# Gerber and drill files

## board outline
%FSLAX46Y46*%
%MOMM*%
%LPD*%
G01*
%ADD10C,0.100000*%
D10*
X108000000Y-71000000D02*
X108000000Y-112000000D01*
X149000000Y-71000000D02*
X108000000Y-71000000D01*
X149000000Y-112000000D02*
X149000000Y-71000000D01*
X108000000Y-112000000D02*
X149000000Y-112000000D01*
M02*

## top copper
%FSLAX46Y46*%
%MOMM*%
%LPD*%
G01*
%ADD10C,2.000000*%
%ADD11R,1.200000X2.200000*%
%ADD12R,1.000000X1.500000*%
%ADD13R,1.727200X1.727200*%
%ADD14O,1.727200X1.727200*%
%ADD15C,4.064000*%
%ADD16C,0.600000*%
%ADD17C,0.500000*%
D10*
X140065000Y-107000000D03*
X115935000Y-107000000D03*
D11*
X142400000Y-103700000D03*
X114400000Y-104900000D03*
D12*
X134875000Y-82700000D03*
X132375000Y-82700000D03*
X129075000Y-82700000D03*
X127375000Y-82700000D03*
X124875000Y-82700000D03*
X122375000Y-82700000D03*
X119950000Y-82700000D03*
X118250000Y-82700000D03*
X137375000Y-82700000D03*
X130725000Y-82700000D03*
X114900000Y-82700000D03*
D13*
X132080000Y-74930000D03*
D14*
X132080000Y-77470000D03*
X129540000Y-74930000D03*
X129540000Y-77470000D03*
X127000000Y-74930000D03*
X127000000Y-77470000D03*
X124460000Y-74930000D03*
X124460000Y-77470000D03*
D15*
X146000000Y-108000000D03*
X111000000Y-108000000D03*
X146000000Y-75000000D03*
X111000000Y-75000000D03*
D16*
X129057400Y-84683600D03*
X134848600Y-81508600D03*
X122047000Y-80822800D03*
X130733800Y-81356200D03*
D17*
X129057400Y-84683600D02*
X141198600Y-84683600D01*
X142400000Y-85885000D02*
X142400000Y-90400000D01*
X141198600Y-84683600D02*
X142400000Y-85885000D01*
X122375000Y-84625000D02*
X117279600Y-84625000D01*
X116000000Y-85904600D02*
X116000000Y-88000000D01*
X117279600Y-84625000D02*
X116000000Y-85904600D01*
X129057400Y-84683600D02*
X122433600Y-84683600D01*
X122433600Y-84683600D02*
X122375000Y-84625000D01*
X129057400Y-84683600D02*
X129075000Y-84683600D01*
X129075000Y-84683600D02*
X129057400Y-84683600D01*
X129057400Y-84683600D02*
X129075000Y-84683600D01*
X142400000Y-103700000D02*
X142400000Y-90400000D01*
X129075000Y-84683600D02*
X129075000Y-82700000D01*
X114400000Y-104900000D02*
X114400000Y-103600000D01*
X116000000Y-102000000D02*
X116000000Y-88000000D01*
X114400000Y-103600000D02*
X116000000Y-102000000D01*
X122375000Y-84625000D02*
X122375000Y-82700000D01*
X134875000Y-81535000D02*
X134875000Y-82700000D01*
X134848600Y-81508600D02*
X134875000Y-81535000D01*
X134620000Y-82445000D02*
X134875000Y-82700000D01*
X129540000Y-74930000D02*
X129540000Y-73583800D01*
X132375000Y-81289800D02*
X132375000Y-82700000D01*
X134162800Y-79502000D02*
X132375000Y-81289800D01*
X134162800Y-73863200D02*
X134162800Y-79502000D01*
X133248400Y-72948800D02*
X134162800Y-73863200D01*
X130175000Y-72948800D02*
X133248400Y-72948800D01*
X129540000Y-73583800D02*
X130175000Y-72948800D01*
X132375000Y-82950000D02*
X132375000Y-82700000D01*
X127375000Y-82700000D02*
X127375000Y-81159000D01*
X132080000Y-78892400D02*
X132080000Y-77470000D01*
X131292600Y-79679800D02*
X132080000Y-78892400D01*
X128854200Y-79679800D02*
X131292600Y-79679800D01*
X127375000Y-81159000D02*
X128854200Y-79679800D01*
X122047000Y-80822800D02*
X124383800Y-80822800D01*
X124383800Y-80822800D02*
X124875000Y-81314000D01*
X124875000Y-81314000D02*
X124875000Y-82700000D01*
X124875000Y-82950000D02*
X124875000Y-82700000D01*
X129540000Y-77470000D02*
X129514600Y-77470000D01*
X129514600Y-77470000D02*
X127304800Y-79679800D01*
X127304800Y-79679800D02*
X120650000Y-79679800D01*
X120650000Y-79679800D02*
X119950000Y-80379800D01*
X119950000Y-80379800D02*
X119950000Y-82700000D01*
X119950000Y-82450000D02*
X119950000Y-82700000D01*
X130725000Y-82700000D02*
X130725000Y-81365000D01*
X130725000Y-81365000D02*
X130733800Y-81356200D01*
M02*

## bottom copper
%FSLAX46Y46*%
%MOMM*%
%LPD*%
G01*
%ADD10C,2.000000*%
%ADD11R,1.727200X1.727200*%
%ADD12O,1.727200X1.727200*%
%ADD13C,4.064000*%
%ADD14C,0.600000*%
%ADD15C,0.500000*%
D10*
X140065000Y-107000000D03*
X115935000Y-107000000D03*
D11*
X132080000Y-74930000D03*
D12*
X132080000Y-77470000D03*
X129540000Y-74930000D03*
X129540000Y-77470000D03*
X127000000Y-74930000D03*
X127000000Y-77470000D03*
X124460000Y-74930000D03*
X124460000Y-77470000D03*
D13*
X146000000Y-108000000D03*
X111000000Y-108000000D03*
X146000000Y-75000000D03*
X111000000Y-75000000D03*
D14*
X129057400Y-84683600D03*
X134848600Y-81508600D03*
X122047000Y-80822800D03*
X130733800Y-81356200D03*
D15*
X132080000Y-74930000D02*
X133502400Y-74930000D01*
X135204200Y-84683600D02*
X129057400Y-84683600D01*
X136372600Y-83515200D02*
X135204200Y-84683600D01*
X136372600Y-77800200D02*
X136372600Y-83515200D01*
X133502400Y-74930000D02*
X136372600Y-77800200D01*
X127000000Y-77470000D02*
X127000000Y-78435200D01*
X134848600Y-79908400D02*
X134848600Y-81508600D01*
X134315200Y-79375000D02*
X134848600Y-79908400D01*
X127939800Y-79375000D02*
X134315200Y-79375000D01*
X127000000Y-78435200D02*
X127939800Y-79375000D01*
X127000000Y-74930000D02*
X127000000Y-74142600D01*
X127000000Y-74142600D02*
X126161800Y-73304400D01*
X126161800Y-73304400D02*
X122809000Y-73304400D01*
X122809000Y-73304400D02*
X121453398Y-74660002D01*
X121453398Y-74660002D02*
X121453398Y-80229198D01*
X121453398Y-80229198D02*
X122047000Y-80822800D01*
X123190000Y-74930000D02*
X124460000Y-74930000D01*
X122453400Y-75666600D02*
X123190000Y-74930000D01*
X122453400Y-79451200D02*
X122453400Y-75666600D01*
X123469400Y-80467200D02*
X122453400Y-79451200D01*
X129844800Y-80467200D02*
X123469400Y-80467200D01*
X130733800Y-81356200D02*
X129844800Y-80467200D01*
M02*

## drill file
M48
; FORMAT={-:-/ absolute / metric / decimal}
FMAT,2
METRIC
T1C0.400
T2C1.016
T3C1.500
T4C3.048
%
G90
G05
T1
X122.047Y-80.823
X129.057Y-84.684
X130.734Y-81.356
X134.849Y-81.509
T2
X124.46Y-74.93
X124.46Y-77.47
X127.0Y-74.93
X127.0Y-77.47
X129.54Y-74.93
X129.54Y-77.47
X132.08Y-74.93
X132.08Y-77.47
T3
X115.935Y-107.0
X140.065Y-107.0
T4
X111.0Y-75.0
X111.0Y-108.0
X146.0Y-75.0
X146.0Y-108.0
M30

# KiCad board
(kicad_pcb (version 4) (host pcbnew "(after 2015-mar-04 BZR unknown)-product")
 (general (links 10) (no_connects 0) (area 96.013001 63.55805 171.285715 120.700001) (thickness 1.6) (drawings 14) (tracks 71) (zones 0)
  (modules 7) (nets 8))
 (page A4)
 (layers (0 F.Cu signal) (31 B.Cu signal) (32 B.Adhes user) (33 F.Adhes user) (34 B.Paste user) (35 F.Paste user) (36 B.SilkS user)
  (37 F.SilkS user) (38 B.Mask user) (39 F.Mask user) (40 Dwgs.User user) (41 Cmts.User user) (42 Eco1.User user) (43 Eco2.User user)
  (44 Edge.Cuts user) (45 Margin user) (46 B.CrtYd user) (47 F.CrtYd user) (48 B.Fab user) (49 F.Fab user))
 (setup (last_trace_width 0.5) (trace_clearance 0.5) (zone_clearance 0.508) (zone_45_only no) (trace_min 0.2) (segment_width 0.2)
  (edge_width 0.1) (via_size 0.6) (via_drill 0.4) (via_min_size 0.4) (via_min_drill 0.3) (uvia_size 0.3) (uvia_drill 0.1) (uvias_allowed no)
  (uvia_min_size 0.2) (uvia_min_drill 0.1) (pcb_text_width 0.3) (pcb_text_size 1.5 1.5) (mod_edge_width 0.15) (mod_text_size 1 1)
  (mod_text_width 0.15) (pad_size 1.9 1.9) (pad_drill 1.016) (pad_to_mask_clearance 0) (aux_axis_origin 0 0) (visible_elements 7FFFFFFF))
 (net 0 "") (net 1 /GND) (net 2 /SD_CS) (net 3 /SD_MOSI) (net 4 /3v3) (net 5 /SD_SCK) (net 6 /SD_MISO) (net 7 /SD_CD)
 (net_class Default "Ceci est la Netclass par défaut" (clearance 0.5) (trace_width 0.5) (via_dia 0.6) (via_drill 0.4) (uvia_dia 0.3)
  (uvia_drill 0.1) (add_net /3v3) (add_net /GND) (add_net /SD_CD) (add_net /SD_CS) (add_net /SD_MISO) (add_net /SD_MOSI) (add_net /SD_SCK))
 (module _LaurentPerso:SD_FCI (layer F.Cu) (at 128 107)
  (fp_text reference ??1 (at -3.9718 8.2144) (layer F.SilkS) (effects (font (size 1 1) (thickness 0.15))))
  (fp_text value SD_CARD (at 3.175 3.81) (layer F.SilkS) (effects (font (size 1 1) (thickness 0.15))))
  (pad "" thru_hole circle (at 12.065 0) (size 2 2) (drill 1.5) (layers *.Cu *.Mask F.SilkS))
  (pad "" thru_hole circle (at -12.065 0) (size 2 2) (drill 1.5) (layers *.Cu *.Mask F.SilkS))
  (pad GND smd rect (at 14.4 -3.3) (size 1.2 2.2) (layers F.Cu F.Paste F.Mask) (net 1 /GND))
  (pad GND smd rect (at -13.6 -2.1) (size 1.2 2.2) (layers F.Cu F.Paste F.Mask) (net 1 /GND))
  (pad 1 smd rect (at 6.875 -24.3) (size 1 1.5) (layers F.Cu F.Paste F.Mask) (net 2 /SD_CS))
  (pad 2 smd rect (at 4.375 -24.3) (size 1 1.5) (layers F.Cu F.Paste F.Mask) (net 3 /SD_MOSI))
  (pad 3 smd rect (at 1.075 -24.3) (size 1 1.5) (layers F.Cu F.Paste F.Mask) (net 1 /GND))
  (pad 4 smd rect (at -0.625 -24.3) (size 1 1.5) (layers F.Cu F.Paste F.Mask) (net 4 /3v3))
  (pad 5 smd rect (at -3.125 -24.3) (size 1 1.5) (layers F.Cu F.Paste F.Mask) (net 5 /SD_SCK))
  (pad 6 smd rect (at -5.625 -24.3) (size 1 1.5) (layers F.Cu F.Paste F.Mask) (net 1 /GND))
  (pad 7 smd rect (at -8.05 -24.3) (size 1 1.5) (layers F.Cu F.Paste F.Mask) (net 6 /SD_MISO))
  (pad 8 smd rect (at -9.75 -24.3) (size 1 1.5) (layers F.Cu F.Paste F.Mask))
  (pad 9 smd rect (at 9.375 -24.3) (size 1 1.5) (layers F.Cu F.Paste F.Mask))
  (pad CD smd rect (at 2.725 -24.3) (size 1 1.5) (layers F.Cu F.Paste F.Mask) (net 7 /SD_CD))
  (pad WP smd rect (at -13.1 -24.3) (size 1 1.5) (layers F.Cu F.Paste F.Mask)))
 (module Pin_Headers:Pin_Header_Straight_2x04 (layer F.Cu) (at 132.08 74.93 270)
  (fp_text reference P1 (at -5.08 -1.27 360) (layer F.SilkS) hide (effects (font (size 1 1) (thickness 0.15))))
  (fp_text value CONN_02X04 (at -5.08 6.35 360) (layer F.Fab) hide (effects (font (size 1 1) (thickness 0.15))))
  (pad 1 thru_hole rect (at 0 0 270) (size 1.7272 1.7272) (drill 1.016) (layers *.Cu *.Mask F.SilkS) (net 1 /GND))
  (pad 2 thru_hole oval (at 2.54 0 270) (size 1.7272 1.7272) (drill 1.016) (layers *.Cu *.Mask F.SilkS) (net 4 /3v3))
  (pad 3 thru_hole oval (at 0 2.54 270) (size 1.7272 1.7272) (drill 1.016) (layers *.Cu *.Mask F.SilkS) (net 3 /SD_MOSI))
  (pad 4 thru_hole oval (at 2.54 2.54 270) (size 1.7272 1.7272) (drill 1.016) (layers *.Cu *.Mask F.SilkS) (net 6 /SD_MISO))
  (pad 5 thru_hole oval (at 0 5.08 270) (size 1.7272 1.7272) (drill 1.016) (layers *.Cu *.Mask F.SilkS) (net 5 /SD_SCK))
  (pad 6 thru_hole oval (at 2.54 5.08 270) (size 1.7272 1.7272) (drill 1.016) (layers *.Cu *.Mask F.SilkS) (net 2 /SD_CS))
  (pad 7 thru_hole oval (at 0 7.62 270) (size 1.7272 1.7272) (drill 1.016) (layers *.Cu *.Mask F.SilkS) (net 7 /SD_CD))
  (pad 8 thru_hole oval (at 2.54 7.62 270) (size 1.7272 1.7272) (drill 1.016) (layers *.Cu *.Mask F.SilkS)))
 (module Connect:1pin (layer F.Cu) (at 146 108)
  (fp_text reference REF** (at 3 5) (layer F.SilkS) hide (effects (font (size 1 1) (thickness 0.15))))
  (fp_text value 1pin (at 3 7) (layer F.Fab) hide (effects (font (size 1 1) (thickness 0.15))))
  (pad 1 thru_hole circle (at 0 0) (size 4.064 4.064) (drill 3.048) (layers *.Cu *.Mask F.SilkS)))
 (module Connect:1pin (layer F.Cu) (at 111 108)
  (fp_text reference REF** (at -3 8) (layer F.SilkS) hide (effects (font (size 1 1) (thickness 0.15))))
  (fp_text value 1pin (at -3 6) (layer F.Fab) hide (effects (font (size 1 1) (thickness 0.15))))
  (pad 1 thru_hole circle (at 0 0) (size 4.064 4.064) (drill 3.048) (layers *.Cu *.Mask F.SilkS)))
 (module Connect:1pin (layer F.Cu) (at 146 75)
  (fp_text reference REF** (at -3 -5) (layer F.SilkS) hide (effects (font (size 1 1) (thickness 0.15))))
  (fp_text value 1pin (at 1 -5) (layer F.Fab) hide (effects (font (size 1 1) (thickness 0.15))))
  (pad 1 thru_hole circle (at 0 0) (size 4.064 4.064) (drill 3.048) (layers *.Cu *.Mask F.SilkS)))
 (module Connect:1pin (layer F.Cu) (at 111 75)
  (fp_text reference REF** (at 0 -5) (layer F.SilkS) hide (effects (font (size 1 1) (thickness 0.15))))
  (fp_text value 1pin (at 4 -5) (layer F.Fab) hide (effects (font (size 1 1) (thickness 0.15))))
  (pad 1 thru_hole circle (at 0 0) (size 4.064 4.064) (drill 3.048) (layers *.Cu *.Mask F.SilkS)))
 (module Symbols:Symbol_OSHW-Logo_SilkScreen (layer F.Cu) (at 128.016 95.631)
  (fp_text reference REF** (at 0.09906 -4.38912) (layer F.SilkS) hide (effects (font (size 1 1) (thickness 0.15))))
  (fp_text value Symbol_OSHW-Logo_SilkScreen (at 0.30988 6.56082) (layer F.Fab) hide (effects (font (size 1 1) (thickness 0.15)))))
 (gr_line (start 108 71) (end 108 112) (angle 90) (layer Edge.Cuts) (width 0.1))
 (gr_line (start 149 71) (end 108 71) (angle 90) (layer Edge.Cuts) (width 0.1))
 (gr_line (start 149 112) (end 149 71) (angle 90) (layer Edge.Cuts) (width 0.1))
 (gr_line (start 108 112) (end 149 112) (angle 90) (layer Edge.Cuts) (width 0.1))
 (segment (start 129.0574 84.6836) (end 141.1986 84.6836) (width 0.5) (layer F.Cu) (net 1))
 (segment (start 142.4 85.885) (end 142.4 90.4) (width 0.5) (layer F.Cu) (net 1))
 (segment (start 141.1986 84.6836) (end 142.4 85.885) (width 0.5) (layer F.Cu) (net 1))
 (segment (start 122.375 84.625) (end 117.2796 84.625) (width 0.5) (layer F.Cu) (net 1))
 (segment (start 116 85.9046) (end 116 88) (width 0.5) (layer F.Cu) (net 1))
 (segment (start 117.2796 84.625) (end 116 85.9046) (width 0.5) (layer F.Cu) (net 1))
 (segment (start 129.0574 84.6836) (end 122.4336 84.6836) (width 0.5) (layer F.Cu) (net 1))
 (segment (start 122.4336 84.6836) (end 122.375 84.625) (width 0.5) (layer F.Cu) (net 1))
 (segment (start 132.08 74.93) (end 133.5024 74.93) (width 0.5) (layer B.Cu) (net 1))
 (via (at 129.0574 84.6836) (size 0.6) (layers F.Cu B.Cu) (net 1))
 (segment (start 135.2042 84.6836) (end 129.0574 84.6836) (width 0.5) (layer B.Cu) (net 1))
 (segment (start 136.3726 83.5152) (end 135.2042 84.6836) (width 0.5) (layer B.Cu) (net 1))
 (segment (start 136.3726 77.8002) (end 136.3726 83.5152) (width 0.5) (layer B.Cu) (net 1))
 (segment (start 133.5024 74.93) (end 136.3726 77.8002) (width 0.5) (layer B.Cu) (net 1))
 (segment (start 129.0574 84.6836) (end 129.075 84.6836) (width 0.5) (layer F.Cu) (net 1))
 (segment (start 129.075 84.6836) (end 129.0574 84.6836) (width 0.5) (layer F.Cu) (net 1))
 (segment (start 129.0574 84.6836) (end 129.075 84.6836) (width 0.5) (layer F.Cu) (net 1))
 (segment (start 142.4 103.7) (end 142.4 90.4) (width 0.5) (layer F.Cu) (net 1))
 (segment (start 129.075 84.6836) (end 129.075 82.7) (width 0.5) (layer F.Cu) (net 1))
 (segment (start 114.4 104.9) (end 114.4 103.6) (width 0.5) (layer F.Cu) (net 1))
 (segment (start 116 102) (end 116 88) (width 0.5) (layer F.Cu) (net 1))
 (segment (start 114.4 103.6) (end 116 102) (width 0.5) (layer F.Cu) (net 1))
 (segment (start 122.375 84.625) (end 122.375 82.7) (width 0.5) (layer F.Cu) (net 1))
 (segment (start 127 77.47) (end 127 78.4352) (width 0.5) (layer B.Cu) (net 2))
 (segment (start 134.875 81.535) (end 134.875 82.7) (width 0.5) (layer F.Cu) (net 2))
 (segment (start 134.8486 81.5086) (end 134.875 81.535) (width 0.5) (layer F.Cu) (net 2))
 (via (at 134.8486 81.5086) (size 0.6) (layers F.Cu B.Cu) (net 2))
 (segment (start 134.8486 79.9084) (end 134.8486 81.5086) (width 0.5) (layer B.Cu) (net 2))
 (segment (start 134.3152 79.375) (end 134.8486 79.9084) (width 0.5) (layer B.Cu) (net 2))
 (segment (start 127.9398 79.375) (end 134.3152 79.375) (width 0.5) (layer B.Cu) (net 2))
 (segment (start 127 78.4352) (end 127.9398 79.375) (width 0.5) (layer B.Cu) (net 2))
 (segment (start 134.62 82.445) (end 134.875 82.7) (width 0.5) (layer F.Cu) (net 2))
 (segment (start 129.54 74.93) (end 129.54 73.5838) (width 0.5) (layer F.Cu) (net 3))
 (segment (start 132.375 81.2898) (end 132.375 82.7) (width 0.5) (layer F.Cu) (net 3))
 (segment (start 134.1628 79.502) (end 132.375 81.2898) (width 0.5) (layer F.Cu) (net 3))
 (segment (start 134.1628 73.8632) (end 134.1628 79.502) (width 0.5) (layer F.Cu) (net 3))
 (segment (start 133.2484 72.9488) (end 134.1628 73.8632) (width 0.5) (layer F.Cu) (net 3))
 (segment (start 130.175 72.9488) (end 133.2484 72.9488) (width 0.5) (layer F.Cu) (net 3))
 (segment (start 129.54 73.5838) (end 130.175 72.9488) (width 0.5) (layer F.Cu) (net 3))
 (segment (start 132.375 82.95) (end 132.375 82.7) (width 0.5) (layer F.Cu) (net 3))
 (segment (start 127.375 82.7) (end 127.375 81.159) (width 0.5) (layer F.Cu) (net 4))
 (segment (start 132.08 78.8924) (end 132.08 77.47) (width 0.5) (layer F.Cu) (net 4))
 (segment (start 131.2926 79.6798) (end 132.08 78.8924) (width 0.5) (layer F.Cu) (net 4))
 (segment (start 128.8542 79.6798) (end 131.2926 79.6798) (width 0.5) (layer F.Cu) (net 4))
 (segment (start 127.375 81.159) (end 128.8542 79.6798) (width 0.5) (layer F.Cu) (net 4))
 (segment (start 127 74.93) (end 127 74.1426) (width 0.5) (layer B.Cu) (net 5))
 (segment (start 127 74.1426) (end 126.1618 73.3044) (width 0.5) (layer B.Cu) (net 5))
 (segment (start 126.1618 73.3044) (end 122.809 73.3044) (width 0.5) (layer B.Cu) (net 5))
 (segment (start 122.809 73.3044) (end 121.453398 74.660002) (width 0.5) (layer B.Cu) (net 5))
 (segment (start 121.453398 74.660002) (end 121.453398 80.229198) (width 0.5) (layer B.Cu) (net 5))
 (segment (start 121.453398 80.229198) (end 122.047 80.8228) (width 0.5) (layer B.Cu) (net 5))
 (via (at 122.047 80.8228) (size 0.6) (layers F.Cu B.Cu) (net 5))
 (segment (start 122.047 80.8228) (end 124.3838 80.8228) (width 0.5) (layer F.Cu) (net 5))
 (segment (start 124.3838 80.8228) (end 124.875 81.314) (width 0.5) (layer F.Cu) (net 5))
 (segment (start 124.875 81.314) (end 124.875 82.7) (width 0.5) (layer F.Cu) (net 5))
 (segment (start 124.875 82.95) (end 124.875 82.7) (width 0.5) (layer F.Cu) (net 5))
 (segment (start 129.54 77.47) (end 129.5146 77.47) (width 0.5) (layer F.Cu) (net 6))
 (segment (start 129.5146 77.47) (end 127.3048 79.6798) (width 0.5) (layer F.Cu) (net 6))
 (segment (start 127.3048 79.6798) (end 120.65 79.6798) (width 0.5) (layer F.Cu) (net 6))
 (segment (start 120.65 79.6798) (end 119.95 80.3798) (width 0.5) (layer F.Cu) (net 6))
 (segment (start 119.95 80.3798) (end 119.95 82.7) (width 0.5) (layer F.Cu) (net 6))
 (segment (start 119.95 82.45) (end 119.95 82.7) (width 0.5) (layer F.Cu) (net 6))
 (segment (start 130.725 82.7) (end 130.725 81.365) (width 0.5) (layer F.Cu) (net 7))
 (segment (start 123.19 74.93) (end 124.46 74.93) (width 0.5) (layer B.Cu) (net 7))
 (segment (start 122.4534 75.6666) (end 123.19 74.93) (width 0.5) (layer B.Cu) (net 7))
 (segment (start 122.4534 79.4512) (end 122.4534 75.6666) (width 0.5) (layer B.Cu) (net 7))
 (segment (start 123.4694 80.4672) (end 122.4534 79.4512) (width 0.5) (layer B.Cu) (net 7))
 (segment (start 129.8448 80.4672) (end 123.4694 80.4672) (width 0.5) (layer B.Cu) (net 7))
 (segment (start 130.7338 81.3562) (end 129.8448 80.4672) (width 0.5) (layer B.Cu) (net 7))
 (via (at 130.7338 81.3562) (size 0.6) (layers F.Cu B.Cu) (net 7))
 (segment (start 130.725 81.365) (end 130.7338 81.3562) (width 0.5) (layer F.Cu) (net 7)))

